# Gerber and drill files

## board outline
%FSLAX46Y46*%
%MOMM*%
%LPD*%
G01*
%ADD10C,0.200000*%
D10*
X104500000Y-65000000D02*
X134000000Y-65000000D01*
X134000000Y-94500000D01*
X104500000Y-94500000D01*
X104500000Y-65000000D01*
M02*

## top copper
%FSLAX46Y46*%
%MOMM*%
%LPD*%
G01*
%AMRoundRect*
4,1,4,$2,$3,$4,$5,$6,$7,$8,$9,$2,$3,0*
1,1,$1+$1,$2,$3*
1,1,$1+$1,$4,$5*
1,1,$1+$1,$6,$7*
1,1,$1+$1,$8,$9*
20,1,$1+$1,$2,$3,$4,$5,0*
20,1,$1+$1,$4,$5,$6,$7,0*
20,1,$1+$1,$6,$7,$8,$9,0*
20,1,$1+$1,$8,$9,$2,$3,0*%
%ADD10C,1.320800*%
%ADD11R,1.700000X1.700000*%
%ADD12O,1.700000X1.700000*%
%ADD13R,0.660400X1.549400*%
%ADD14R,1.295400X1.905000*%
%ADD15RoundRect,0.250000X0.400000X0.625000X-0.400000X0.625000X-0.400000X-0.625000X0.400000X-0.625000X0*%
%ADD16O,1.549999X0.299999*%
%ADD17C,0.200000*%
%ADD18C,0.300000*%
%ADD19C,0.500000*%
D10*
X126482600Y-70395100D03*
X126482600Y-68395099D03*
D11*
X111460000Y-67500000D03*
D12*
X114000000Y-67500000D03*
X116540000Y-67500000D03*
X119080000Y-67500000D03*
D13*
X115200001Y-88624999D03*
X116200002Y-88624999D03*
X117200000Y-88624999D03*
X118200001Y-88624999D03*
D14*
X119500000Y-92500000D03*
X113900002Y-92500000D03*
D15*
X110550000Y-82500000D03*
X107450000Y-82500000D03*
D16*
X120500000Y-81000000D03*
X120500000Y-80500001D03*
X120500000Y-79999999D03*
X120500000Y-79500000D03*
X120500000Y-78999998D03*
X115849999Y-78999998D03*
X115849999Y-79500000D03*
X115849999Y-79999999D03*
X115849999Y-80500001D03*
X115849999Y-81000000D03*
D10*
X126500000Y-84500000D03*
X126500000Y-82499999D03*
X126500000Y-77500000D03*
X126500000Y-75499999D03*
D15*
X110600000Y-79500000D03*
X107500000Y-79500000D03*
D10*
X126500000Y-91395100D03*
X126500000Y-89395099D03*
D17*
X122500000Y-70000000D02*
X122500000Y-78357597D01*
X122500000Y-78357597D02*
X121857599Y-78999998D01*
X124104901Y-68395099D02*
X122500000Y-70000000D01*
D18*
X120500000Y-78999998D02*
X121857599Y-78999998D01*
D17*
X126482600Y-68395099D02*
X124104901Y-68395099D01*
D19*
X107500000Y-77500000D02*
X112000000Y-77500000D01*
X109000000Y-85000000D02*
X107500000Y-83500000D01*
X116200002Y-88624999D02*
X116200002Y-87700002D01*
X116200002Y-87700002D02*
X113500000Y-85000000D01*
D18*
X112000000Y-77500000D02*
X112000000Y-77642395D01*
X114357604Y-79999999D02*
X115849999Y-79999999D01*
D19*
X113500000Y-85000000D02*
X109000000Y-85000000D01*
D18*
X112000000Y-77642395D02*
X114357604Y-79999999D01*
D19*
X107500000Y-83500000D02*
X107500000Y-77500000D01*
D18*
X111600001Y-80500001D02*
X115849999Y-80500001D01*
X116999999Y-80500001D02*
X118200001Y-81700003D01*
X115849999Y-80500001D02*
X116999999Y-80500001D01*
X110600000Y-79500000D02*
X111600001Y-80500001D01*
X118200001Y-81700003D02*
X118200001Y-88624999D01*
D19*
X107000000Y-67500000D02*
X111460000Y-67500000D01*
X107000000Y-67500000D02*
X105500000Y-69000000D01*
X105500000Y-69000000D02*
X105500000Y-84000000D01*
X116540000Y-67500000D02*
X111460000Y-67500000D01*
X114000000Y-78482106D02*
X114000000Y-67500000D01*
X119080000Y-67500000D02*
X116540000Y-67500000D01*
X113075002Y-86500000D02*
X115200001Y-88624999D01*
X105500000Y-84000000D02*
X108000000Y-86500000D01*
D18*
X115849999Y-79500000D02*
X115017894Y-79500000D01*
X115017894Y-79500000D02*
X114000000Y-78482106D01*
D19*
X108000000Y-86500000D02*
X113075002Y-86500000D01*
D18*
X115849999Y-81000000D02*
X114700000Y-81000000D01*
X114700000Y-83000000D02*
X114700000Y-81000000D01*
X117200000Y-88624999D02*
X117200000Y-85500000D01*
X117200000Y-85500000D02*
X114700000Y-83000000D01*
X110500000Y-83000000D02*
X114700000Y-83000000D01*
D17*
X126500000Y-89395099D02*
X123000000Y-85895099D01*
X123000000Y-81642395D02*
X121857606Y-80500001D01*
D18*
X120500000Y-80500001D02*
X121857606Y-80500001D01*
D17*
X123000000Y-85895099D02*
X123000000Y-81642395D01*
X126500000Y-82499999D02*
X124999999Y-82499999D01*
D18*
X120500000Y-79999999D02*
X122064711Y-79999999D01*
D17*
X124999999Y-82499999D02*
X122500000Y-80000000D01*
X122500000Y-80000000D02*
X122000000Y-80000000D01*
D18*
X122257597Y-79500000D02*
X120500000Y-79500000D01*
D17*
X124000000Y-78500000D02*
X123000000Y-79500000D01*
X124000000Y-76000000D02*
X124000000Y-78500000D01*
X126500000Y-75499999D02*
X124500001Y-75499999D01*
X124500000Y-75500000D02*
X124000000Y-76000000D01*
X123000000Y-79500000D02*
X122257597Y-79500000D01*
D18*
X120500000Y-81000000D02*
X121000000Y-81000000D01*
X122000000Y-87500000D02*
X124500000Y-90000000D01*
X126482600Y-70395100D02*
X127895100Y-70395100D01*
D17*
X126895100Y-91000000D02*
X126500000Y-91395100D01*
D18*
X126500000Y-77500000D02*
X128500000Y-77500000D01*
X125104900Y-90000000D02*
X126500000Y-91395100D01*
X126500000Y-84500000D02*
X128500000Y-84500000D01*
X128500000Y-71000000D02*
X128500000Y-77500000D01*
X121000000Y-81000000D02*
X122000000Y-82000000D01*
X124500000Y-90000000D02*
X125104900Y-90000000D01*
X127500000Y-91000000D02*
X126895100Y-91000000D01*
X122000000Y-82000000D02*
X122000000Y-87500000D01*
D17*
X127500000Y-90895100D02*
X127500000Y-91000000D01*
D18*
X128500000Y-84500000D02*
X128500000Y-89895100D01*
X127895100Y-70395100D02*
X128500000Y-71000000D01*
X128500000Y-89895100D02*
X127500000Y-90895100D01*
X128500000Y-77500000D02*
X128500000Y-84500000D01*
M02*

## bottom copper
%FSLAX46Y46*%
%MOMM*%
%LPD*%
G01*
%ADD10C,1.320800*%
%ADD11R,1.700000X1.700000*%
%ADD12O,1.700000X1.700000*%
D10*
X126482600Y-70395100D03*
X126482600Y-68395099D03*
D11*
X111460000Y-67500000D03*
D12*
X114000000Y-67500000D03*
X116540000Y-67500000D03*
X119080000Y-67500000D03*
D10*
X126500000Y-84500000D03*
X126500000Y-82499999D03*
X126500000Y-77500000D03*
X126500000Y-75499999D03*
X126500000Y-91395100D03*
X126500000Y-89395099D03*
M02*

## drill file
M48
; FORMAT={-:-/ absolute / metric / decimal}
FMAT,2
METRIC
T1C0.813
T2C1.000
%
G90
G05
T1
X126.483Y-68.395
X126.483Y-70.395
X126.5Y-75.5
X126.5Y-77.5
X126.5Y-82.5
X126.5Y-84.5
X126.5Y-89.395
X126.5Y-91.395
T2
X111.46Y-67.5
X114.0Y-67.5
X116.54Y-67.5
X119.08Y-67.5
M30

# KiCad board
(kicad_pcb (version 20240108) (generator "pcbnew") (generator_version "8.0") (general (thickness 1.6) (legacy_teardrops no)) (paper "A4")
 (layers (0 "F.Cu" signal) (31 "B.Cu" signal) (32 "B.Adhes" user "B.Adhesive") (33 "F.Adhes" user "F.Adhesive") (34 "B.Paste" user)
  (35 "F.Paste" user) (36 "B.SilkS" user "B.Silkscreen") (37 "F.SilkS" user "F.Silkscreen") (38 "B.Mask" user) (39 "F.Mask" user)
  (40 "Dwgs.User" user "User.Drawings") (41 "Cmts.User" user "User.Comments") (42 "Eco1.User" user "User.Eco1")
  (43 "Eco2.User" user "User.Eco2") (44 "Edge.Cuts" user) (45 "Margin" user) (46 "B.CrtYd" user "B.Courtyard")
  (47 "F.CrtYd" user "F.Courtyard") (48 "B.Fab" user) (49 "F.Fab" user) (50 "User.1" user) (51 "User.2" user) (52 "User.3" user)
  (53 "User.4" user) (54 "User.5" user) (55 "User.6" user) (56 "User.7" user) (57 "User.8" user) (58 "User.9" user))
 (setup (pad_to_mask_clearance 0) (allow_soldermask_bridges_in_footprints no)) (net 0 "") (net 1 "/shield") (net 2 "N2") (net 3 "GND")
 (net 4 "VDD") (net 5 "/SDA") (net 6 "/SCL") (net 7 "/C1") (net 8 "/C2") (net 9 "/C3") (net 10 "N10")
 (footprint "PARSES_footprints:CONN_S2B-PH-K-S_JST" (layer "F.Cu") (at 126.4826 70.3951 90)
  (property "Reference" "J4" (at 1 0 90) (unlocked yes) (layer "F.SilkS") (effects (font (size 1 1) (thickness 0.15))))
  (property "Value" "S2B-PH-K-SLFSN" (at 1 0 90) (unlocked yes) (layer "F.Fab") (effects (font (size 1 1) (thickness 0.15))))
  (pad "1" thru_hole circle (at 0 0 90) (size 1.3208 1.3208) (drill 0.8128) (layers "*.Cu" "*.Mask") (remove_unused_layers no)
   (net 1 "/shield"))
  (pad "2" thru_hole circle (at 2.000001 0 90) (size 1.3208 1.3208) (drill 0.8128) (layers "*.Cu" "*.Mask") (remove_unused_layers no)
   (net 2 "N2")))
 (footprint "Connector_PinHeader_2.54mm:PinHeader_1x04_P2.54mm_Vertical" (layer "F.Cu") (at 111.46 67.5 90)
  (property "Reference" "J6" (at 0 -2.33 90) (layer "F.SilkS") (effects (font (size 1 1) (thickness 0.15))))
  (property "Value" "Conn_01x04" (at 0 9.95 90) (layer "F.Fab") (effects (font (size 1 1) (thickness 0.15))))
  (pad "1" thru_hole rect (at 0 0 90) (size 1.7 1.7) (drill 1) (layers "*.Cu" "*.Mask") (remove_unused_layers no) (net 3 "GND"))
  (pad "2" thru_hole oval (at 0 2.54 90) (size 1.7 1.7) (drill 1) (layers "*.Cu" "*.Mask") (remove_unused_layers no) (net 3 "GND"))
  (pad "3" thru_hole oval (at 0 5.08 90) (size 1.7 1.7) (drill 1) (layers "*.Cu" "*.Mask") (remove_unused_layers no) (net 3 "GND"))
  (pad "4" thru_hole oval (at 0 7.62 90) (size 1.7 1.7) (drill 1) (layers "*.Cu" "*.Mask") (remove_unused_layers no) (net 3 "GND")))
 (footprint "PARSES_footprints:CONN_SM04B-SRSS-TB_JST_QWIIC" (layer "F.Cu") (at 116.700001 90.723499 180)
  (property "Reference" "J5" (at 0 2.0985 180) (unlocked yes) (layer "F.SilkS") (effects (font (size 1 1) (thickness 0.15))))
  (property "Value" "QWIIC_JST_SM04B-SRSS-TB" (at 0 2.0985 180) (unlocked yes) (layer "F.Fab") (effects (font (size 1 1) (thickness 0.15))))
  (pad "1" smd rect (at 1.5 2.0985 180) (size 0.6604 1.5494) (layers "F.Cu" "F.Paste" "F.Mask") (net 3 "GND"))
  (pad "2" smd rect (at 0.499999 2.0985 180) (size 0.6604 1.5494) (layers "F.Cu" "F.Paste" "F.Mask") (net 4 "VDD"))
  (pad "3" smd rect (at -0.499999 2.0985 180) (size 0.6604 1.5494) (layers "F.Cu" "F.Paste" "F.Mask") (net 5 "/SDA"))
  (pad "4" smd rect (at -1.5 2.0985 180) (size 0.6604 1.5494) (layers "F.Cu" "F.Paste" "F.Mask") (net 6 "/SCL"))
  (pad "5" smd rect (at -2.799999 -1.776501 270) (size 1.905 1.2954) (layers "F.Cu" "F.Paste" "F.Mask"))
  (pad "6" smd rect (at 2.799999 -1.776501 270) (size 1.905 1.2954) (layers "F.Cu" "F.Paste" "F.Mask")))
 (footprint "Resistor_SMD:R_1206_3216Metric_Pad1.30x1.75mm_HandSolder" (layer "F.Cu") (at 109 82.5 180)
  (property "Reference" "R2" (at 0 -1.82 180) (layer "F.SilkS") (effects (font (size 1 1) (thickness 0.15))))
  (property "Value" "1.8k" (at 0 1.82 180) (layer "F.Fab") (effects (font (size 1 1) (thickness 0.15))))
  (pad "1" smd roundrect (at -1.55 0 180) (size 1.3 1.75) (layers "F.Cu" "F.Paste" "F.Mask") (roundrect_rratio 0.192308) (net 5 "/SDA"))
  (pad "2" smd roundrect (at 1.55 0 180) (size 1.3 1.75) (layers "F.Cu" "F.Paste" "F.Mask") (roundrect_rratio 0.192308) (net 4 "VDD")))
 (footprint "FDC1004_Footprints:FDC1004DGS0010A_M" (layer "F.Cu") (at 118.175001 79.999999 180)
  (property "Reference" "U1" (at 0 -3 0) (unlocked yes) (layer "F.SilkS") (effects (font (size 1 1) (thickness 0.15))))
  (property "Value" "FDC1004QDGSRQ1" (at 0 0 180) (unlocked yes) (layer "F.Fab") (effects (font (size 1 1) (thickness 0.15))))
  (pad "1" smd oval (at -2.324999 -1.000001 270) (size 0.299999 1.549999) (layers "F.Cu" "F.Paste" "F.Mask") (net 1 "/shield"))
  (pad "2" smd oval (at -2.324999 -0.500002 270) (size 0.299999 1.549999) (layers "F.Cu" "F.Paste" "F.Mask") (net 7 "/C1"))
  (pad "3" smd oval (at -2.324999 0 270) (size 0.299999 1.549999) (layers "F.Cu" "F.Paste" "F.Mask") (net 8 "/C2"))
  (pad "4" smd oval (at -2.324999 0.499999 270) (size 0.299999 1.549999) (layers "F.Cu" "F.Paste" "F.Mask") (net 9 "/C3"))
  (pad "5" smd oval (at -2.324999 1.000001 270) (size 0.299999 1.549999) (layers "F.Cu" "F.Paste" "F.Mask") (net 2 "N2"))
  (pad "6" smd oval (at 2.325002 1.000001 270) (size 0.299999 1.549999) (layers "F.Cu" "F.Paste" "F.Mask") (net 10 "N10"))
  (pad "7" smd oval (at 2.325002 0.499999 270) (size 0.299999 1.549999) (layers "F.Cu" "F.Paste" "F.Mask") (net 3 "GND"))
  (pad "8" smd oval (at 2.325002 0 270) (size 0.299999 1.549999) (layers "F.Cu" "F.Paste" "F.Mask") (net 4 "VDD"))
  (pad "9" smd oval (at 2.325002 -0.500002 270) (size 0.299999 1.549999) (layers "F.Cu" "F.Paste" "F.Mask") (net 6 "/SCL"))
  (pad "10" smd oval (at 2.325002 -1.000001 270) (size 0.299999 1.549999) (layers "F.Cu" "F.Paste" "F.Mask") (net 5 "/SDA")))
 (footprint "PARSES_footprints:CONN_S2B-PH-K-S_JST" (layer "F.Cu") (at 126.5 84.5 90)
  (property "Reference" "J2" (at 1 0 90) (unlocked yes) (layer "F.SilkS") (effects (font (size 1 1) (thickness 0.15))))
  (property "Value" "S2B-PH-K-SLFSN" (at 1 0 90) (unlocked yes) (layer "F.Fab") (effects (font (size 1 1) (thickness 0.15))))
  (pad "1" thru_hole circle (at 0 0 90) (size 1.3208 1.3208) (drill 0.8128) (layers "*.Cu" "*.Mask") (remove_unused_layers no)
   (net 1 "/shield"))
  (pad "2" thru_hole circle (at 2.000001 0 90) (size 1.3208 1.3208) (drill 0.8128) (layers "*.Cu" "*.Mask") (remove_unused_layers no)
   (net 8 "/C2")))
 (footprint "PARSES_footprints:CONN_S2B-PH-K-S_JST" (layer "F.Cu") (at 126.5 77.5 90)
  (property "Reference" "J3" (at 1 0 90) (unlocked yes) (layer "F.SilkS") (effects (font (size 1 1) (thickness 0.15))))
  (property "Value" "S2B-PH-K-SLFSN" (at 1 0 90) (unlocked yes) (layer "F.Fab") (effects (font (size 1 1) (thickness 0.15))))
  (pad "1" thru_hole circle (at 0 0 90) (size 1.3208 1.3208) (drill 0.8128) (layers "*.Cu" "*.Mask") (remove_unused_layers no)
   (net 1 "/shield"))
  (pad "2" thru_hole circle (at 2.000001 0 90) (size 1.3208 1.3208) (drill 0.8128) (layers "*.Cu" "*.Mask") (remove_unused_layers no)
   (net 9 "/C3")))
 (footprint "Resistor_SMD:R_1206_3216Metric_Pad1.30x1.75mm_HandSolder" (layer "F.Cu") (at 109.05 79.5 180)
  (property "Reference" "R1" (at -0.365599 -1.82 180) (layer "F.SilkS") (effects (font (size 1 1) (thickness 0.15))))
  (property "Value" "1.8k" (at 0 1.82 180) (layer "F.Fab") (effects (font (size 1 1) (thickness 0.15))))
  (pad "1" smd roundrect (at -1.55 0 180) (size 1.3 1.75) (layers "F.Cu" "F.Paste" "F.Mask") (roundrect_rratio 0.192308) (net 6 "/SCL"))
  (pad "2" smd roundrect (at 1.55 0 180) (size 1.3 1.75) (layers "F.Cu" "F.Paste" "F.Mask") (roundrect_rratio 0.192308) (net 4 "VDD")))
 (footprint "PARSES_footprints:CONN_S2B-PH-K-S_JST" (layer "F.Cu") (at 126.5 91.3951 90)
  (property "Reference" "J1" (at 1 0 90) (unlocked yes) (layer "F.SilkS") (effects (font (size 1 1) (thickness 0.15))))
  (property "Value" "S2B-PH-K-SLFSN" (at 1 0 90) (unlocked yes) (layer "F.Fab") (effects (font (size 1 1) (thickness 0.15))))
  (pad "1" thru_hole circle (at 0 0 90) (size 1.3208 1.3208) (drill 0.8128) (layers "*.Cu" "*.Mask") (remove_unused_layers no)
   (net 1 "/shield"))
  (pad "2" thru_hole circle (at 2.000001 0 90) (size 1.3208 1.3208) (drill 0.8128) (layers "*.Cu" "*.Mask") (remove_unused_layers no)
   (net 7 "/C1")))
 (gr_rect (start 104.5 65) (end 134 94.5) (stroke (width 0.2) (type default)) (fill none) (layer "Edge.Cuts"))
 (segment (start 122.5 70) (end 122.5 78.357597) (width 0.2) (layer "F.Cu") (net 2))
 (segment (start 122.5 78.357597) (end 121.857599 78.999998) (width 0.2) (layer "F.Cu") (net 2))
 (segment (start 124.104901 68.395099) (end 122.5 70) (width 0.2) (layer "F.Cu") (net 2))
 (segment (start 120.5 78.999998) (end 121.857599 78.999998) (width 0.3) (layer "F.Cu") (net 2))
 (segment (start 126.4826 68.395099) (end 124.104901 68.395099) (width 0.2) (layer "F.Cu") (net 2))
 (segment (start 107.5 77.5) (end 112 77.5) (width 0.5) (layer "F.Cu") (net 4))
 (segment (start 109 85) (end 107.5 83.5) (width 0.5) (layer "F.Cu") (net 4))
 (segment (start 116.200002 88.624999) (end 116.200002 87.700002) (width 0.5) (layer "F.Cu") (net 4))
 (segment (start 116.200002 87.700002) (end 113.5 85) (width 0.5) (layer "F.Cu") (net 4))
 (segment (start 112 77.5) (end 112 77.642395) (width 0.3) (layer "F.Cu") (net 4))
 (segment (start 114.357604 79.999999) (end 115.849999 79.999999) (width 0.3) (layer "F.Cu") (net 4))
 (segment (start 113.5 85) (end 109 85) (width 0.5) (layer "F.Cu") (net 4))
 (segment (start 112 77.642395) (end 114.357604 79.999999) (width 0.3) (layer "F.Cu") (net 4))
 (segment (start 107.5 83.5) (end 107.5 77.5) (width 0.5) (layer "F.Cu") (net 4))
 (segment (start 111.600001 80.500001) (end 115.849999 80.500001) (width 0.3) (layer "F.Cu") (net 6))
 (segment (start 116.999999 80.500001) (end 118.200001 81.700003) (width 0.3) (layer "F.Cu") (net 6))
 (segment (start 115.849999 80.500001) (end 116.999999 80.500001) (width 0.3) (layer "F.Cu") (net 6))
 (segment (start 110.6 79.5) (end 111.600001 80.500001) (width 0.3) (layer "F.Cu") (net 6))
 (segment (start 118.200001 81.700003) (end 118.200001 88.624999) (width 0.3) (layer "F.Cu") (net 6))
 (segment (start 107 67.5) (end 111.46 67.5) (width 0.5) (layer "F.Cu") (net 3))
 (segment (start 107 67.5) (end 105.5 69) (width 0.5) (layer "F.Cu") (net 3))
 (segment (start 105.5 69) (end 105.5 84) (width 0.5) (layer "F.Cu") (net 3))
 (segment (start 116.54 67.5) (end 111.46 67.5) (width 0.5) (layer "F.Cu") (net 3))
 (segment (start 114 78.482106) (end 114 67.5) (width 0.5) (layer "F.Cu") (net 3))
 (segment (start 119.08 67.5) (end 116.54 67.5) (width 0.5) (layer "F.Cu") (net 3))
 (segment (start 113.075002 86.5) (end 115.200001 88.624999) (width 0.5) (layer "F.Cu") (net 3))
 (segment (start 105.5 84) (end 108 86.5) (width 0.5) (layer "F.Cu") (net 3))
 (segment (start 115.849999 79.5) (end 115.017894 79.5) (width 0.3) (layer "F.Cu") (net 3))
 (segment (start 115.017894 79.5) (end 114 78.482106) (width 0.3) (layer "F.Cu") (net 3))
 (segment (start 108 86.5) (end 113.075002 86.5) (width 0.5) (layer "F.Cu") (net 3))
 (segment (start 115.849999 81) (end 114.7 81) (width 0.3) (layer "F.Cu") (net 5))
 (segment (start 114.7 83) (end 114.7 81) (width 0.3) (layer "F.Cu") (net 5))
 (segment (start 117.2 88.624999) (end 117.2 85.5) (width 0.3) (layer "F.Cu") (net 5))
 (segment (start 117.2 85.5) (end 114.7 83) (width 0.3) (layer "F.Cu") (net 5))
 (segment (start 110.5 83) (end 114.7 83) (width 0.3) (layer "F.Cu") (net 5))
 (segment (start 126.5 89.395099) (end 123 85.895099) (width 0.2) (layer "F.Cu") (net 7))
 (segment (start 123 81.642395) (end 121.857606 80.500001) (width 0.2) (layer "F.Cu") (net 7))
 (segment (start 120.5 80.500001) (end 121.857606 80.500001) (width 0.3) (layer "F.Cu") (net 7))
 (segment (start 123 85.895099) (end 123 81.642395) (width 0.2) (layer "F.Cu") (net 7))
 (segment (start 126.5 82.499999) (end 124.999999 82.499999) (width 0.2) (layer "F.Cu") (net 8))
 (segment (start 120.5 79.999999) (end 122.064711 79.999999) (width 0.3) (layer "F.Cu") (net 8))
 (segment (start 124.999999 82.499999) (end 122.5 80) (width 0.2) (layer "F.Cu") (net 8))
 (segment (start 122.5 80) (end 122 80) (width 0.2) (layer "F.Cu") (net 8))
 (segment (start 122.257597 79.5) (end 120.5 79.5) (width 0.3) (layer "F.Cu") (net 9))
 (segment (start 124 78.5) (end 123 79.5) (width 0.2) (layer "F.Cu") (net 9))
 (segment (start 124 76) (end 124 78.5) (width 0.2) (layer "F.Cu") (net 9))
 (segment (start 126.5 75.499999) (end 124.500001 75.499999) (width 0.2) (layer "F.Cu") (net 9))
 (segment (start 124.5 75.5) (end 124 76) (width 0.2) (layer "F.Cu") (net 9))
 (segment (start 123 79.5) (end 122.257597 79.5) (width 0.2) (layer "F.Cu") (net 9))
 (segment (start 120.5 81) (end 121 81) (width 0.3) (layer "F.Cu") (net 1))
 (segment (start 122 87.5) (end 124.5 90) (width 0.3) (layer "F.Cu") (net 1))
 (segment (start 126.4826 70.3951) (end 127.8951 70.3951) (width 0.3) (layer "F.Cu") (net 1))
 (segment (start 126.8951 91) (end 126.5 91.3951) (width 0.2) (layer "F.Cu") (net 1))
 (segment (start 126.5 77.5) (end 128.5 77.5) (width 0.3) (layer "F.Cu") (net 1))
 (segment (start 125.1049 90) (end 126.5 91.3951) (width 0.3) (layer "F.Cu") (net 1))
 (segment (start 126.5 84.5) (end 128.5 84.5) (width 0.3) (layer "F.Cu") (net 1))
 (segment (start 128.5 71) (end 128.5 77.5) (width 0.3) (layer "F.Cu") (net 1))
 (segment (start 121 81) (end 122 82) (width 0.3) (layer "F.Cu") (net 1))
 (segment (start 124.5 90) (end 125.1049 90) (width 0.3) (layer "F.Cu") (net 1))
 (segment (start 127.5 91) (end 126.8951 91) (width 0.3) (layer "F.Cu") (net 1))
 (segment (start 122 82) (end 122 87.5) (width 0.3) (layer "F.Cu") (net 1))
 (segment (start 127.5 90.8951) (end 127.5 91) (width 0.2) (layer "F.Cu") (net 1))
 (segment (start 128.5 84.5) (end 128.5 89.8951) (width 0.3) (layer "F.Cu") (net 1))
 (segment (start 127.8951 70.3951) (end 128.5 71) (width 0.3) (layer "F.Cu") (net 1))
 (segment (start 128.5 89.8951) (end 127.5 90.8951) (width 0.3) (layer "F.Cu") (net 1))
 (segment (start 128.5 77.5) (end 128.5 84.5) (width 0.3) (layer "F.Cu") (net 1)))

